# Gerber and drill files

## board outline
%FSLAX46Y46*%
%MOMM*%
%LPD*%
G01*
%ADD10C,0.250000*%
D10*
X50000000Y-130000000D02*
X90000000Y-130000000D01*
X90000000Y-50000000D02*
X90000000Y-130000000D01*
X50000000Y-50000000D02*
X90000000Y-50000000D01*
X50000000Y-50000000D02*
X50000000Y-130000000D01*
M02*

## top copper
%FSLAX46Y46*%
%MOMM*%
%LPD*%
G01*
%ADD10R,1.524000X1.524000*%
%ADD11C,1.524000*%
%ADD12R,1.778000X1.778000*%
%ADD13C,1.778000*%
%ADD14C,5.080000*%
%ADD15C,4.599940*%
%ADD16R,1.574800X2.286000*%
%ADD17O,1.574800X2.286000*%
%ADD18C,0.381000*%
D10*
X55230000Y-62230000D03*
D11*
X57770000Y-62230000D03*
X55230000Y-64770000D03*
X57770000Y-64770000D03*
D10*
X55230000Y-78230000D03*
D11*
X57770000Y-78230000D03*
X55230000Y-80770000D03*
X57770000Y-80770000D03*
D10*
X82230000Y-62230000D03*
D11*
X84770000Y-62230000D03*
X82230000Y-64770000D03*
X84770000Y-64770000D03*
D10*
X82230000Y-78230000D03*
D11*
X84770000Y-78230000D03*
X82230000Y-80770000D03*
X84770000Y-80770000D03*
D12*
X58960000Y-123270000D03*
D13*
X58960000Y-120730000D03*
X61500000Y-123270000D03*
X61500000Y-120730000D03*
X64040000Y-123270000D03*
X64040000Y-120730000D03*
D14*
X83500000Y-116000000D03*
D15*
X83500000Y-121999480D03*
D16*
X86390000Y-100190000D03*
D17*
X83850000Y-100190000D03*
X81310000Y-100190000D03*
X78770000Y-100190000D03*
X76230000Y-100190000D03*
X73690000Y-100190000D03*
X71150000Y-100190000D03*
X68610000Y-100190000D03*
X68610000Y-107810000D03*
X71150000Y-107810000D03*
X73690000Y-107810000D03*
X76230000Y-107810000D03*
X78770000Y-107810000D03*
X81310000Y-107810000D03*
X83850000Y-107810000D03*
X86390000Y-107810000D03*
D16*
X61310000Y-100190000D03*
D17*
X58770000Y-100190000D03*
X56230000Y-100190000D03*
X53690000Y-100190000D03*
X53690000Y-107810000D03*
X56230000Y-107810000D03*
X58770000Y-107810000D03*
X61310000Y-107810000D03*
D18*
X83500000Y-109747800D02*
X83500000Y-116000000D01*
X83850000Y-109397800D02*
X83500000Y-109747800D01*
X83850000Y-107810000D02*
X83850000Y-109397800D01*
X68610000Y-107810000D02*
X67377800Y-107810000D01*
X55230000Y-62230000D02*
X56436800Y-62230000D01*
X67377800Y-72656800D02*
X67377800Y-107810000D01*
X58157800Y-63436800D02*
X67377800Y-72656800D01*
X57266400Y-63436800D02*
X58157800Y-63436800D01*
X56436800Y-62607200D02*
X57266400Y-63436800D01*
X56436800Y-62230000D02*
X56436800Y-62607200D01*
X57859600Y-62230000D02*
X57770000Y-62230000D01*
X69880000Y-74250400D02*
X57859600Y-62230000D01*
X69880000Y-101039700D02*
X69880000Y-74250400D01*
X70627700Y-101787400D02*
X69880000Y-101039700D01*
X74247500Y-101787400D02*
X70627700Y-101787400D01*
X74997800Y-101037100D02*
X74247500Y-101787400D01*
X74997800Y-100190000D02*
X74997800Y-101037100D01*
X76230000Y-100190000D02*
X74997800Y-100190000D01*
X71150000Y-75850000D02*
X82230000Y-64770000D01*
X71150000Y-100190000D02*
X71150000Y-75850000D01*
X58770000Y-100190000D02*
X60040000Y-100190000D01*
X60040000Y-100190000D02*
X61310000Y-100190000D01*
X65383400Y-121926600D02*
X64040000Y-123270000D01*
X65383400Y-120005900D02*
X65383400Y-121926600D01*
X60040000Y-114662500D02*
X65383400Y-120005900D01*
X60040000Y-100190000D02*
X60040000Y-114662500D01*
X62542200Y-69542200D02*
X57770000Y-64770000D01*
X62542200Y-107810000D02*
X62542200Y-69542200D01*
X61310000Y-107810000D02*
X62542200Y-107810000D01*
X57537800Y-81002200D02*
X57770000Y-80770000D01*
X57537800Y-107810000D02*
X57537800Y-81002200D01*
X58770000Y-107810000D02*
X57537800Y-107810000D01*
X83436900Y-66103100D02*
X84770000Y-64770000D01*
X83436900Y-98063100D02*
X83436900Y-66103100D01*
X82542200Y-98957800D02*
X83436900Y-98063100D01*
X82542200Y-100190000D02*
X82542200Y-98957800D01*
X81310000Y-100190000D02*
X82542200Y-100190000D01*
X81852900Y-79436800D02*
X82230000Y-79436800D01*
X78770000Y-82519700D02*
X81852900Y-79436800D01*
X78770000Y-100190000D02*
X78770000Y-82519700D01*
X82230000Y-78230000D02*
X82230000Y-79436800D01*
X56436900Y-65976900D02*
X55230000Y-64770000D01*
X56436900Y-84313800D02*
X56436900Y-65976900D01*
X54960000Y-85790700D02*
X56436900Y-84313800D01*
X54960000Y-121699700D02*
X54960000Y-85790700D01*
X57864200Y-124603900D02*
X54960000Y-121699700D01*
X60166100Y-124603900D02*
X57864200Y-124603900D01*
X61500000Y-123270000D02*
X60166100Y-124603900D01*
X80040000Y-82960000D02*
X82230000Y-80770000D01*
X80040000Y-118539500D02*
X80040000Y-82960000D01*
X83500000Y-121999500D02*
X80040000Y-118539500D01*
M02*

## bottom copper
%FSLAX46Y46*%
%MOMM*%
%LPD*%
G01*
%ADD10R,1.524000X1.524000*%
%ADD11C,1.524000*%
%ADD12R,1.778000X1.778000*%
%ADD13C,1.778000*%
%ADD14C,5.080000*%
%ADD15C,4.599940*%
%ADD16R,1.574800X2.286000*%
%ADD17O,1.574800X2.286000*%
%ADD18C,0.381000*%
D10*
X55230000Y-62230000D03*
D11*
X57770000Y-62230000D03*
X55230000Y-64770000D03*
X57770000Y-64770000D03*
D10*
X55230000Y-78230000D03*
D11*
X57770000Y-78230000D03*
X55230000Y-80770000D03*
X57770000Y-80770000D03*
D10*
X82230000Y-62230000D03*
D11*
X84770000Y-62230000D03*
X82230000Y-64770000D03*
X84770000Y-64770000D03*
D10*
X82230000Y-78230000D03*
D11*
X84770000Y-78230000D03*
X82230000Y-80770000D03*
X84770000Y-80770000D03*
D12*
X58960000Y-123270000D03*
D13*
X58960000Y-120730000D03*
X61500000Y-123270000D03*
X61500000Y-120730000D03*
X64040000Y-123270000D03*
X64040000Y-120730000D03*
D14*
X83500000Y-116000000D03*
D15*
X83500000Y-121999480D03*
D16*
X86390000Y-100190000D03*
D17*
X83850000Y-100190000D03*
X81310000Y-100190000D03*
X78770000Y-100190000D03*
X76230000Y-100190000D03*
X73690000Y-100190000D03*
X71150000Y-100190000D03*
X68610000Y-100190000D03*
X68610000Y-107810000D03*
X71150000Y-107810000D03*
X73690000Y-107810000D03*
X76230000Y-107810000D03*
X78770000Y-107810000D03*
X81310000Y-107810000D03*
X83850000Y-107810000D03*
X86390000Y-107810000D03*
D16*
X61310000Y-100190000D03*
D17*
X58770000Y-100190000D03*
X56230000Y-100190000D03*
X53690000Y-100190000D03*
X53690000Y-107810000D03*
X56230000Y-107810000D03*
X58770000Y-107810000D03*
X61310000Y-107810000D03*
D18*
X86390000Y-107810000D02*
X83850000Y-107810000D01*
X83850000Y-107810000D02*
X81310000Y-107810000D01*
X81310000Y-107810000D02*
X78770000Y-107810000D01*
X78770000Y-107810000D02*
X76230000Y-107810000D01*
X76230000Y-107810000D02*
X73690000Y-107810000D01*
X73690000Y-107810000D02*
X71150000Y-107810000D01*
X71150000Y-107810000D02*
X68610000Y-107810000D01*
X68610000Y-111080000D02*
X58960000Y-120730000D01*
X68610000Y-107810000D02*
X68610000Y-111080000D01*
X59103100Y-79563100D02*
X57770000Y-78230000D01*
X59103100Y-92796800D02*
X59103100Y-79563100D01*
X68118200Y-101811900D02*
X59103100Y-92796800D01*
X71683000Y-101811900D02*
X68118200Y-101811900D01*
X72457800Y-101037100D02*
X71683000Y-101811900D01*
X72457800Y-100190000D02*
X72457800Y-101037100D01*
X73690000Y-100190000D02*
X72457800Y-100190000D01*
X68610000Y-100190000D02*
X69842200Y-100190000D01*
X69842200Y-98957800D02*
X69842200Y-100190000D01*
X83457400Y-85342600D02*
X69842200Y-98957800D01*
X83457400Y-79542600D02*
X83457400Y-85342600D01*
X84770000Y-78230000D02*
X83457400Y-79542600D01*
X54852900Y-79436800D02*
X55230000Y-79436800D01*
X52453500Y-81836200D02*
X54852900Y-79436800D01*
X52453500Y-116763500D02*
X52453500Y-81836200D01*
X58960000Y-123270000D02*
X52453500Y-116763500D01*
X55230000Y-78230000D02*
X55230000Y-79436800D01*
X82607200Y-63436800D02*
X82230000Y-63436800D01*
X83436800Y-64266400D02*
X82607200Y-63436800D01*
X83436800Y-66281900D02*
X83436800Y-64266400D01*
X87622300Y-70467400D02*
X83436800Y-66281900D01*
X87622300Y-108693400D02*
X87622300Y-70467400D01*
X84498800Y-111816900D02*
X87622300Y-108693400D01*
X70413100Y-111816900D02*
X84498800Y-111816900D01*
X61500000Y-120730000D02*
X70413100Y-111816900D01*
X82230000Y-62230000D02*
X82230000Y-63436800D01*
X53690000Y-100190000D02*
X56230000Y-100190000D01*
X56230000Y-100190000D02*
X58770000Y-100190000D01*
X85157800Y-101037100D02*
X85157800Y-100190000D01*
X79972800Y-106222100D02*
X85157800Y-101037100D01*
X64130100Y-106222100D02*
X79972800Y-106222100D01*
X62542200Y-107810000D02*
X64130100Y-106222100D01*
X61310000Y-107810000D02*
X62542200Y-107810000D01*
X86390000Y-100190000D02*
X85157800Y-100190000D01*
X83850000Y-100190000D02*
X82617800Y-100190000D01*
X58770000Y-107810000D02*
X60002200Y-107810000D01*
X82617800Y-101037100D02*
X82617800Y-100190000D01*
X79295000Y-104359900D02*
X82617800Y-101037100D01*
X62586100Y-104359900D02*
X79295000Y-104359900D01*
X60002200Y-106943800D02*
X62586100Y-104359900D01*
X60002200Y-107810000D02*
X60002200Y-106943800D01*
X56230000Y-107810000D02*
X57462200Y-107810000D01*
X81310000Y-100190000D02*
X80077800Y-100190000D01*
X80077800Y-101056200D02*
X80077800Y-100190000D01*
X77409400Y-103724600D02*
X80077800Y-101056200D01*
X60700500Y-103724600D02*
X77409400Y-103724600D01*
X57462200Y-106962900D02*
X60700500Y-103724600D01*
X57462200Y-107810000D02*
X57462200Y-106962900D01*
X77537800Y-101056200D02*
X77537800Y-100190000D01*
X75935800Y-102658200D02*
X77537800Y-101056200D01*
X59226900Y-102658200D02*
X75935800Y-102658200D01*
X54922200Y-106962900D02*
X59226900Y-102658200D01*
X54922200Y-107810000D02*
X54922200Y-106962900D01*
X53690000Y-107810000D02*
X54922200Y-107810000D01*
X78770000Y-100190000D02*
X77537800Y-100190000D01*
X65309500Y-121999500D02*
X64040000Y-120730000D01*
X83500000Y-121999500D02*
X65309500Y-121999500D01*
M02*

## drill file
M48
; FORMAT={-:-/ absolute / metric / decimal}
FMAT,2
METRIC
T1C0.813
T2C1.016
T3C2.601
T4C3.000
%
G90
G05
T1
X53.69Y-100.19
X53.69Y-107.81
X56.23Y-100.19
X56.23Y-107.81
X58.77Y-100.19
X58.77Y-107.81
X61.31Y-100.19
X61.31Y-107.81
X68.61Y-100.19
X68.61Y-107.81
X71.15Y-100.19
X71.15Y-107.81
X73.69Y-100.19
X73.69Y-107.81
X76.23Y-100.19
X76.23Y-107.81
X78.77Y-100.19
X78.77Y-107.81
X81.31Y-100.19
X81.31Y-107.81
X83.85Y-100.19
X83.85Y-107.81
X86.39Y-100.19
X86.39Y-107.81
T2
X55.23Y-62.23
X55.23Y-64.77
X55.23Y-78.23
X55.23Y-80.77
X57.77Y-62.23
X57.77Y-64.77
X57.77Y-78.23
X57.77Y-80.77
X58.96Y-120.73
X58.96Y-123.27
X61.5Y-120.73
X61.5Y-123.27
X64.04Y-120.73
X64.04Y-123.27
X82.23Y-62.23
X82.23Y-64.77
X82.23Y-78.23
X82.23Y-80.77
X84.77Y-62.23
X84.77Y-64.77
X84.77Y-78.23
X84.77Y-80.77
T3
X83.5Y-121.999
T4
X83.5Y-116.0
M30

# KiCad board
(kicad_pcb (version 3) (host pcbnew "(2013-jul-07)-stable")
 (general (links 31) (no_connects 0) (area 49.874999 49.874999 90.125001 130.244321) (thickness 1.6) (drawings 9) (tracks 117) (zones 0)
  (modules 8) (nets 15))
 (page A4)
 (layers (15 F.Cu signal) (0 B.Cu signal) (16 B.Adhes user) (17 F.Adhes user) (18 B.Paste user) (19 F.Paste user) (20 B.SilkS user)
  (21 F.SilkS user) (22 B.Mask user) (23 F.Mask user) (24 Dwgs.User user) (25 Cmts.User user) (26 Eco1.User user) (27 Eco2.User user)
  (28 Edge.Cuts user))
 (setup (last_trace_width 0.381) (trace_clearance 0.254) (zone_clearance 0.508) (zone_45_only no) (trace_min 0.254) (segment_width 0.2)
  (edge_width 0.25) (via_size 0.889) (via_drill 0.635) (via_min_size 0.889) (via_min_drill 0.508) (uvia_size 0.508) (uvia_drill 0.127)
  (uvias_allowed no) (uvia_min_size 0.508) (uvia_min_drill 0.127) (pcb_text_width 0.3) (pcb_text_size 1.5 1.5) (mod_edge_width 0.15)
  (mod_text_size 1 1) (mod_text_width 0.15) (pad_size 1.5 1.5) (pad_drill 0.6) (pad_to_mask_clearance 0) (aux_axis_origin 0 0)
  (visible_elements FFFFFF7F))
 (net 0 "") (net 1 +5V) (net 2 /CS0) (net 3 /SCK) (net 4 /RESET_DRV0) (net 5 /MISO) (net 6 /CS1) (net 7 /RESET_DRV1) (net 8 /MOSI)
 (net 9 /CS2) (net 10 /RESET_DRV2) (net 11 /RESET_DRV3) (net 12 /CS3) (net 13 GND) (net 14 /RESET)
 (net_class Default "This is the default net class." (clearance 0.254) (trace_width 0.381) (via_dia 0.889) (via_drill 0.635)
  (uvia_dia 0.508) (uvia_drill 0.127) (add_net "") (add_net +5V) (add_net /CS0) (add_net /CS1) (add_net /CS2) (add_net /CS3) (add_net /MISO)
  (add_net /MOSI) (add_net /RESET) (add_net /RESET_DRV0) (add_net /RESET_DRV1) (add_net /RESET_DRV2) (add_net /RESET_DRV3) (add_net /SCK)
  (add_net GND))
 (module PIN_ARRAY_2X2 (layer F.Cu) (at 56.5 63.5 270)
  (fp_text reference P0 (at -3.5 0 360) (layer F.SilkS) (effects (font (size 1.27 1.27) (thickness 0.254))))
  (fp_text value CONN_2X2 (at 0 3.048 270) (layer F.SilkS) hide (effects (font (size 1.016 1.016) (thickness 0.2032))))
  (pad 1 thru_hole rect (at -1.27 1.27 270) (size 1.524 1.524) (drill 1.016) (layers *.Cu *.Mask F.SilkS) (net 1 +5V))
  (pad 2 thru_hole circle (at -1.27 -1.27 270) (size 1.524 1.524) (drill 1.016) (layers *.Cu *.Mask F.SilkS) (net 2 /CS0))
  (pad 3 thru_hole circle (at 1.27 1.27 270) (size 1.524 1.524) (drill 1.016) (layers *.Cu *.Mask F.SilkS) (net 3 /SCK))
  (pad 4 thru_hole circle (at 1.27 -1.27 270) (size 1.524 1.524) (drill 1.016) (layers *.Cu *.Mask F.SilkS) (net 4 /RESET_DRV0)))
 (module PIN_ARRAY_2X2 (layer F.Cu) (at 56.5 79.5 270)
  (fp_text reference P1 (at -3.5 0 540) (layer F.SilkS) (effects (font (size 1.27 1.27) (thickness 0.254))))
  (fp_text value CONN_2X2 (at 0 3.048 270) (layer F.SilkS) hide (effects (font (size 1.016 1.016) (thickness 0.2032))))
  (pad 1 thru_hole rect (at -1.27 1.27 270) (size 1.524 1.524) (drill 1.016) (layers *.Cu *.Mask F.SilkS) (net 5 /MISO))
  (pad 2 thru_hole circle (at -1.27 -1.27 270) (size 1.524 1.524) (drill 1.016) (layers *.Cu *.Mask F.SilkS) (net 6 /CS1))
  (pad 3 thru_hole circle (at 1.27 1.27 270) (size 1.524 1.524) (drill 1.016) (layers *.Cu *.Mask F.SilkS))
  (pad 4 thru_hole circle (at 1.27 -1.27 270) (size 1.524 1.524) (drill 1.016) (layers *.Cu *.Mask F.SilkS) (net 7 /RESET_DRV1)))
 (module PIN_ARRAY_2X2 (layer F.Cu) (at 83.5 63.5 270)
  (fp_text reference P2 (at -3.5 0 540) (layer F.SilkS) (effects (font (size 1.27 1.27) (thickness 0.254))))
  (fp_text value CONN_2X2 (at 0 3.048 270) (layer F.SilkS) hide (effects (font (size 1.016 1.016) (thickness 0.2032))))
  (pad 1 thru_hole rect (at -1.27 1.27 270) (size 1.524 1.524) (drill 1.016) (layers *.Cu *.Mask F.SilkS) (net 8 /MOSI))
  (pad 2 thru_hole circle (at -1.27 -1.27 270) (size 1.524 1.524) (drill 1.016) (layers *.Cu *.Mask F.SilkS))
  (pad 3 thru_hole circle (at 1.27 1.27 270) (size 1.524 1.524) (drill 1.016) (layers *.Cu *.Mask F.SilkS) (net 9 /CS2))
  (pad 4 thru_hole circle (at 1.27 -1.27 270) (size 1.524 1.524) (drill 1.016) (layers *.Cu *.Mask F.SilkS) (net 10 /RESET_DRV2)))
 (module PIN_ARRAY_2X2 (layer F.Cu) (at 83.5 79.5 270)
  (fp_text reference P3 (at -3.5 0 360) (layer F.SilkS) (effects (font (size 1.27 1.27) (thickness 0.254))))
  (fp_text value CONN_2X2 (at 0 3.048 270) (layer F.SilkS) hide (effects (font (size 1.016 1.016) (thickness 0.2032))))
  (pad 1 thru_hole rect (at -1.27 1.27 270) (size 1.524 1.524) (drill 1.016) (layers *.Cu *.Mask F.SilkS) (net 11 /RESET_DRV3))
  (pad 2 thru_hole circle (at -1.27 -1.27 270) (size 1.524 1.524) (drill 1.016) (layers *.Cu *.Mask F.SilkS) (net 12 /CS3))
  (pad 3 thru_hole circle (at 1.27 1.27 270) (size 1.524 1.524) (drill 1.016) (layers *.Cu *.Mask F.SilkS) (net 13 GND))
  (pad 4 thru_hole circle (at 1.27 -1.27 270) (size 1.524 1.524) (drill 1.016) (layers *.Cu *.Mask F.SilkS)))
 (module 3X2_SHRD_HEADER (layer F.Cu) (at 61.5 122)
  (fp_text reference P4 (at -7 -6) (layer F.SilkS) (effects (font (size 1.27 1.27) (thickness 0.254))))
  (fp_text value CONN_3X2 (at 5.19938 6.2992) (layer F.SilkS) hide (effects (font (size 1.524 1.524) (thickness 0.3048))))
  (pad 1 thru_hole rect (at -2.54 1.27) (size 1.778 1.778) (drill 1.016) (layers *.Cu *.Mask F.SilkS) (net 5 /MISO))
  (pad 2 thru_hole circle (at -2.54 -1.27) (size 1.778 1.778) (drill 1.016) (layers *.Cu *.Mask F.SilkS) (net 1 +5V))
  (pad 3 thru_hole circle (at 0 1.27) (size 1.778 1.778) (drill 1.016) (layers *.Cu *.Mask F.SilkS) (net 3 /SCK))
  (pad 4 thru_hole circle (at 0 -1.27) (size 1.778 1.778) (drill 1.016) (layers *.Cu *.Mask F.SilkS) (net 8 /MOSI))
  (pad 5 thru_hole circle (at 2.54 1.27) (size 1.778 1.778) (drill 1.016) (layers *.Cu *.Mask F.SilkS) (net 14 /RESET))
  (pad 6 thru_hole circle (at 2.54 -1.27) (size 1.778 1.778) (drill 1.016) (layers *.Cu *.Mask F.SilkS) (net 13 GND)))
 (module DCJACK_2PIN (layer F.Cu) (at 83.5 116 270)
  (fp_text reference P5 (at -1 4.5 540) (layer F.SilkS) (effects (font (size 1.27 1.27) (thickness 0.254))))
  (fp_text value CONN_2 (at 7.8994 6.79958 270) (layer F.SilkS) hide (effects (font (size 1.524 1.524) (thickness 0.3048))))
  (pad 1 thru_hole circle (at 0 0 270) (size 5.08 5.08) (drill 2.99974) (layers *.Cu *.Mask F.SilkS) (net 1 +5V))
  (pad 2 thru_hole circle (at 5.99948 0 270) (size 4.59994 4.59994) (drill 2.60096) (layers *.Cu *.Mask F.SilkS) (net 13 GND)))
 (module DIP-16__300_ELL (layer F.Cu) (at 77.5 104 180)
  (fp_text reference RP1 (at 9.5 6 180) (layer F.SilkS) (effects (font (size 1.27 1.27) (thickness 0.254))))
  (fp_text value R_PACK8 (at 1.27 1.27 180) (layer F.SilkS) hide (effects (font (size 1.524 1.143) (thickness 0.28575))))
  (pad 1 thru_hole rect (at -8.89 3.81 180) (size 1.5748 2.286) (drill 0.8128) (layers *.Cu *.Mask F.SilkS) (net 4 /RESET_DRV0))
  (pad 2 thru_hole oval (at -6.35 3.81 180) (size 1.5748 2.286) (drill 0.8128) (layers *.Cu *.Mask F.SilkS) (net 7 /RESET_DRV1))
  (pad 3 thru_hole oval (at -3.81 3.81 180) (size 1.5748 2.286) (drill 0.8128) (layers *.Cu *.Mask F.SilkS) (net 10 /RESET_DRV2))
  (pad 4 thru_hole oval (at -1.27 3.81 180) (size 1.5748 2.286) (drill 0.8128) (layers *.Cu *.Mask F.SilkS) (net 11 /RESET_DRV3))
  (pad 5 thru_hole oval (at 1.27 3.81 180) (size 1.5748 2.286) (drill 0.8128) (layers *.Cu *.Mask F.SilkS) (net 2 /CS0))
  (pad 6 thru_hole oval (at 3.81 3.81 180) (size 1.5748 2.286) (drill 0.8128) (layers *.Cu *.Mask F.SilkS) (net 6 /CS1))
  (pad 7 thru_hole oval (at 6.35 3.81 180) (size 1.5748 2.286) (drill 0.8128) (layers *.Cu *.Mask F.SilkS) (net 9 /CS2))
  (pad 8 thru_hole oval (at 8.89 3.81 180) (size 1.5748 2.286) (drill 0.8128) (layers *.Cu *.Mask F.SilkS) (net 12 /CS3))
  (pad 9 thru_hole oval (at 8.89 -3.81 180) (size 1.5748 2.286) (drill 0.8128) (layers *.Cu *.Mask F.SilkS) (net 1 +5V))
  (pad 10 thru_hole oval (at 6.35 -3.81 180) (size 1.5748 2.286) (drill 0.8128) (layers *.Cu *.Mask F.SilkS) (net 1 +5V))
  (pad 11 thru_hole oval (at 3.81 -3.81 180) (size 1.5748 2.286) (drill 0.8128) (layers *.Cu *.Mask F.SilkS) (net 1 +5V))
  (pad 12 thru_hole oval (at 1.27 -3.81 180) (size 1.5748 2.286) (drill 0.8128) (layers *.Cu *.Mask F.SilkS) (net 1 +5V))
  (pad 13 thru_hole oval (at -1.27 -3.81 180) (size 1.5748 2.286) (drill 0.8128) (layers *.Cu *.Mask F.SilkS) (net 1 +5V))
  (pad 14 thru_hole oval (at -3.81 -3.81 180) (size 1.5748 2.286) (drill 0.8128) (layers *.Cu *.Mask F.SilkS) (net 1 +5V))
  (pad 15 thru_hole oval (at -6.35 -3.81 180) (size 1.5748 2.286) (drill 0.8128) (layers *.Cu *.Mask F.SilkS) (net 1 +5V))
  (pad 16 thru_hole oval (at -8.89 -3.81 180) (size 1.5748 2.286) (drill 0.8128) (layers *.Cu *.Mask F.SilkS) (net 1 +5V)))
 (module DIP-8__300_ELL (layer F.Cu) (at 57.5 104 180)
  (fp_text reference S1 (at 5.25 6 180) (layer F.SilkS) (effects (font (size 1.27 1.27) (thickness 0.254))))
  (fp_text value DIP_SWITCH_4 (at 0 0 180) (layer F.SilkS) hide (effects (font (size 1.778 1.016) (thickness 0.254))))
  (pad 1 thru_hole rect (at -3.81 3.81 180) (size 1.5748 2.286) (drill 0.8128) (layers *.Cu *.Mask F.SilkS) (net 14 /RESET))
  (pad 2 thru_hole oval (at -1.27 3.81 180) (size 1.5748 2.286) (drill 0.8128) (layers *.Cu *.Mask F.SilkS) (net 14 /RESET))
  (pad 3 thru_hole oval (at 1.27 3.81 180) (size 1.5748 2.286) (drill 0.8128) (layers *.Cu *.Mask F.SilkS) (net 14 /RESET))
  (pad 4 thru_hole oval (at 3.81 3.81 180) (size 1.5748 2.286) (drill 0.8128) (layers *.Cu *.Mask F.SilkS) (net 14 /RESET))
  (pad 5 thru_hole oval (at 3.81 -3.81 180) (size 1.5748 2.286) (drill 0.8128) (layers *.Cu *.Mask F.SilkS) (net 11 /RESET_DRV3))
  (pad 6 thru_hole oval (at 1.27 -3.81 180) (size 1.5748 2.286) (drill 0.8128) (layers *.Cu *.Mask F.SilkS) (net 10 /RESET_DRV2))
  (pad 7 thru_hole oval (at -1.27 -3.81 180) (size 1.5748 2.286) (drill 0.8128) (layers *.Cu *.Mask F.SilkS) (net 7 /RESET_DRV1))
  (pad 8 thru_hole oval (at -3.81 -3.81 180) (size 1.5748 2.286) (drill 0.8128) (layers *.Cu *.Mask F.SilkS) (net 4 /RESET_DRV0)))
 (gr_line (start 50 130) (end 90 130) (angle 90) (layer Edge.Cuts) (width 0.25))
 (gr_line (start 90 50) (end 90 130) (angle 90) (layer Edge.Cuts) (width 0.25))
 (gr_line (start 50 50) (end 90 50) (angle 90) (layer Edge.Cuts) (width 0.25))
 (gr_line (start 50 50) (end 50 130) (angle 90) (layer Edge.Cuts) (width 0.25))
 (segment (start 86.39 107.81) (end 83.85 107.81) (width 0.381) (layer B.Cu) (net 1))
 (segment (start 83.85 107.81) (end 81.31 107.81) (width 0.381) (layer B.Cu) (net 1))
 (segment (start 81.31 107.81) (end 78.77 107.81) (width 0.381) (layer B.Cu) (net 1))
 (segment (start 78.77 107.81) (end 76.23 107.81) (width 0.381) (layer B.Cu) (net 1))
 (segment (start 76.23 107.81) (end 73.69 107.81) (width 0.381) (layer B.Cu) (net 1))
 (segment (start 73.69 107.81) (end 71.15 107.81) (width 0.381) (layer B.Cu) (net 1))
 (segment (start 83.5 109.7478) (end 83.5 116) (width 0.381) (layer F.Cu) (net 1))
 (segment (start 83.85 109.3978) (end 83.5 109.7478) (width 0.381) (layer F.Cu) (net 1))
 (segment (start 83.85 107.81) (end 83.85 109.3978) (width 0.381) (layer F.Cu) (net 1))
 (segment (start 71.15 107.81) (end 68.61 107.81) (width 0.381) (layer B.Cu) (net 1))
 (segment (start 68.61 111.08) (end 58.96 120.73) (width 0.381) (layer B.Cu) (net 1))
 (segment (start 68.61 107.81) (end 68.61 111.08) (width 0.381) (layer B.Cu) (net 1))
 (segment (start 68.61 107.81) (end 67.3778 107.81) (width 0.381) (layer F.Cu) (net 1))
 (segment (start 55.23 62.23) (end 56.4368 62.23) (width 0.381) (layer F.Cu) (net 1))
 (segment (start 67.3778 72.6568) (end 67.3778 107.81) (width 0.381) (layer F.Cu) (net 1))
 (segment (start 58.1578 63.4368) (end 67.3778 72.6568) (width 0.381) (layer F.Cu) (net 1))
 (segment (start 57.2664 63.4368) (end 58.1578 63.4368) (width 0.381) (layer F.Cu) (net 1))
 (segment (start 56.4368 62.6072) (end 57.2664 63.4368) (width 0.381) (layer F.Cu) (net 1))
 (segment (start 56.4368 62.23) (end 56.4368 62.6072) (width 0.381) (layer F.Cu) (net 1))
 (segment (start 57.8596 62.23) (end 57.77 62.23) (width 0.381) (layer F.Cu) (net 2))
 (segment (start 69.88 74.2504) (end 57.8596 62.23) (width 0.381) (layer F.Cu) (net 2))
 (segment (start 69.88 101.0397) (end 69.88 74.2504) (width 0.381) (layer F.Cu) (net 2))
 (segment (start 70.6277 101.7874) (end 69.88 101.0397) (width 0.381) (layer F.Cu) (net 2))
 (segment (start 74.2475 101.7874) (end 70.6277 101.7874) (width 0.381) (layer F.Cu) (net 2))
 (segment (start 74.9978 101.0371) (end 74.2475 101.7874) (width 0.381) (layer F.Cu) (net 2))
 (segment (start 74.9978 100.19) (end 74.9978 101.0371) (width 0.381) (layer F.Cu) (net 2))
 (segment (start 76.23 100.19) (end 74.9978 100.19) (width 0.381) (layer F.Cu) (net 2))
 (segment (start 59.1031 79.5631) (end 57.77 78.23) (width 0.381) (layer B.Cu) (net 6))
 (segment (start 59.1031 92.7968) (end 59.1031 79.5631) (width 0.381) (layer B.Cu) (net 6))
 (segment (start 68.1182 101.8119) (end 59.1031 92.7968) (width 0.381) (layer B.Cu) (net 6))
 (segment (start 71.683 101.8119) (end 68.1182 101.8119) (width 0.381) (layer B.Cu) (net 6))
 (segment (start 72.4578 101.0371) (end 71.683 101.8119) (width 0.381) (layer B.Cu) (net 6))
 (segment (start 72.4578 100.19) (end 72.4578 101.0371) (width 0.381) (layer B.Cu) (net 6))
 (segment (start 73.69 100.19) (end 72.4578 100.19) (width 0.381) (layer B.Cu) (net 6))
 (segment (start 71.15 75.85) (end 82.23 64.77) (width 0.381) (layer F.Cu) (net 9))
 (segment (start 71.15 100.19) (end 71.15 75.85) (width 0.381) (layer F.Cu) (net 9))
 (segment (start 68.61 100.19) (end 69.8422 100.19) (width 0.381) (layer B.Cu) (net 12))
 (segment (start 69.8422 98.9578) (end 69.8422 100.19) (width 0.381) (layer B.Cu) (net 12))
 (segment (start 83.4574 85.3426) (end 69.8422 98.9578) (width 0.381) (layer B.Cu) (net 12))
 (segment (start 83.4574 79.5426) (end 83.4574 85.3426) (width 0.381) (layer B.Cu) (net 12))
 (segment (start 84.77 78.23) (end 83.4574 79.5426) (width 0.381) (layer B.Cu) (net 12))
 (segment (start 54.8529 79.4368) (end 55.23 79.4368) (width 0.381) (layer B.Cu) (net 5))
 (segment (start 52.4535 81.8362) (end 54.8529 79.4368) (width 0.381) (layer B.Cu) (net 5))
 (segment (start 52.4535 116.7635) (end 52.4535 81.8362) (width 0.381) (layer B.Cu) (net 5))
 (segment (start 58.96 123.27) (end 52.4535 116.7635) (width 0.381) (layer B.Cu) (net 5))
 (segment (start 55.23 78.23) (end 55.23 79.4368) (width 0.381) (layer B.Cu) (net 5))
 (segment (start 82.6072 63.4368) (end 82.23 63.4368) (width 0.381) (layer B.Cu) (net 8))
 (segment (start 83.4368 64.2664) (end 82.6072 63.4368) (width 0.381) (layer B.Cu) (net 8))
 (segment (start 83.4368 66.2819) (end 83.4368 64.2664) (width 0.381) (layer B.Cu) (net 8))
 (segment (start 87.6223 70.4674) (end 83.4368 66.2819) (width 0.381) (layer B.Cu) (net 8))
 (segment (start 87.6223 108.6934) (end 87.6223 70.4674) (width 0.381) (layer B.Cu) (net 8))
 (segment (start 84.4988 111.8169) (end 87.6223 108.6934) (width 0.381) (layer B.Cu) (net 8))
 (segment (start 70.4131 111.8169) (end 84.4988 111.8169) (width 0.381) (layer B.Cu) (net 8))
 (segment (start 61.5 120.73) (end 70.4131 111.8169) (width 0.381) (layer B.Cu) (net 8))
 (segment (start 82.23 62.23) (end 82.23 63.4368) (width 0.381) (layer B.Cu) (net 8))
 (segment (start 53.69 100.19) (end 56.23 100.19) (width 0.381) (layer B.Cu) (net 14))
 (segment (start 56.23 100.19) (end 58.77 100.19) (width 0.381) (layer B.Cu) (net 14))
 (segment (start 58.77 100.19) (end 60.04 100.19) (width 0.381) (layer F.Cu) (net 14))
 (segment (start 60.04 100.19) (end 61.31 100.19) (width 0.381) (layer F.Cu) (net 14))
 (segment (start 65.3834 121.9266) (end 64.04 123.27) (width 0.381) (layer F.Cu) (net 14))
 (segment (start 65.3834 120.0059) (end 65.3834 121.9266) (width 0.381) (layer F.Cu) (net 14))
 (segment (start 60.04 114.6625) (end 65.3834 120.0059) (width 0.381) (layer F.Cu) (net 14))
 (segment (start 60.04 100.19) (end 60.04 114.6625) (width 0.381) (layer F.Cu) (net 14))
 (segment (start 62.5422 69.5422) (end 57.77 64.77) (width 0.381) (layer F.Cu) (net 4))
 (segment (start 62.5422 107.81) (end 62.5422 69.5422) (width 0.381) (layer F.Cu) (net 4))
 (segment (start 61.31 107.81) (end 62.5422 107.81) (width 0.381) (layer F.Cu) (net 4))
 (segment (start 85.1578 101.0371) (end 85.1578 100.19) (width 0.381) (layer B.Cu) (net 4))
 (segment (start 79.9728 106.2221) (end 85.1578 101.0371) (width 0.381) (layer B.Cu) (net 4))
 (segment (start 64.1301 106.2221) (end 79.9728 106.2221) (width 0.381) (layer B.Cu) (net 4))
 (segment (start 62.5422 107.81) (end 64.1301 106.2221) (width 0.381) (layer B.Cu) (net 4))
 (segment (start 61.31 107.81) (end 62.5422 107.81) (width 0.381) (layer B.Cu) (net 4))
 (segment (start 86.39 100.19) (end 85.1578 100.19) (width 0.381) (layer B.Cu) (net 4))
 (segment (start 57.5378 81.0022) (end 57.77 80.77) (width 0.381) (layer F.Cu) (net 7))
 (segment (start 57.5378 107.81) (end 57.5378 81.0022) (width 0.381) (layer F.Cu) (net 7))
 (segment (start 58.77 107.81) (end 57.5378 107.81) (width 0.381) (layer F.Cu) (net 7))
 (segment (start 83.85 100.19) (end 82.6178 100.19) (width 0.381) (layer B.Cu) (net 7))
 (segment (start 58.77 107.81) (end 60.0022 107.81) (width 0.381) (layer B.Cu) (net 7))
 (segment (start 82.6178 101.0371) (end 82.6178 100.19) (width 0.381) (layer B.Cu) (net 7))
 (segment (start 79.295 104.3599) (end 82.6178 101.0371) (width 0.381) (layer B.Cu) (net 7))
 (segment (start 62.5861 104.3599) (end 79.295 104.3599) (width 0.381) (layer B.Cu) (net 7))
 (segment (start 60.0022 106.9438) (end 62.5861 104.3599) (width 0.381) (layer B.Cu) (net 7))
 (segment (start 60.0022 107.81) (end 60.0022 106.9438) (width 0.381) (layer B.Cu) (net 7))
 (segment (start 56.23 107.81) (end 57.4622 107.81) (width 0.381) (layer B.Cu) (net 10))
 (segment (start 81.31 100.19) (end 80.0778 100.19) (width 0.381) (layer B.Cu) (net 10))
 (segment (start 83.4369 66.1031) (end 84.77 64.77) (width 0.381) (layer F.Cu) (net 10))
 (segment (start 83.4369 98.0631) (end 83.4369 66.1031) (width 0.381) (layer F.Cu) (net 10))
 (segment (start 82.5422 98.9578) (end 83.4369 98.0631) (width 0.381) (layer F.Cu) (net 10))
 (segment (start 82.5422 100.19) (end 82.5422 98.9578) (width 0.381) (layer F.Cu) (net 10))
 (segment (start 81.31 100.19) (end 82.5422 100.19) (width 0.381) (layer F.Cu) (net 10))
 (segment (start 80.0778 101.0562) (end 80.0778 100.19) (width 0.381) (layer B.Cu) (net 10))
 (segment (start 77.4094 103.7246) (end 80.0778 101.0562) (width 0.381) (layer B.Cu) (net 10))
 (segment (start 60.7005 103.7246) (end 77.4094 103.7246) (width 0.381) (layer B.Cu) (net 10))
 (segment (start 57.4622 106.9629) (end 60.7005 103.7246) (width 0.381) (layer B.Cu) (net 10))
 (segment (start 57.4622 107.81) (end 57.4622 106.9629) (width 0.381) (layer B.Cu) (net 10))
 (segment (start 81.8529 79.4368) (end 82.23 79.4368) (width 0.381) (layer F.Cu) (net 11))
 (segment (start 78.77 82.5197) (end 81.8529 79.4368) (width 0.381) (layer F.Cu) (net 11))
 (segment (start 78.77 100.19) (end 78.77 82.5197) (width 0.381) (layer F.Cu) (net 11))
 (segment (start 82.23 78.23) (end 82.23 79.4368) (width 0.381) (layer F.Cu) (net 11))
 (segment (start 77.5378 101.0562) (end 77.5378 100.19) (width 0.381) (layer B.Cu) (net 11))
 (segment (start 75.9358 102.6582) (end 77.5378 101.0562) (width 0.381) (layer B.Cu) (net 11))
 (segment (start 59.2269 102.6582) (end 75.9358 102.6582) (width 0.381) (layer B.Cu) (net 11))
 (segment (start 54.9222 106.9629) (end 59.2269 102.6582) (width 0.381) (layer B.Cu) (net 11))
 (segment (start 54.9222 107.81) (end 54.9222 106.9629) (width 0.381) (layer B.Cu) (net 11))
 (segment (start 53.69 107.81) (end 54.9222 107.81) (width 0.381) (layer B.Cu) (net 11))
 (segment (start 78.77 100.19) (end 77.5378 100.19) (width 0.381) (layer B.Cu) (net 11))
 (segment (start 56.4369 65.9769) (end 55.23 64.77) (width 0.381) (layer F.Cu) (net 3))
 (segment (start 56.4369 84.3138) (end 56.4369 65.9769) (width 0.381) (layer F.Cu) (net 3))
 (segment (start 54.96 85.7907) (end 56.4369 84.3138) (width 0.381) (layer F.Cu) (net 3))
 (segment (start 54.96 121.6997) (end 54.96 85.7907) (width 0.381) (layer F.Cu) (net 3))
 (segment (start 57.8642 124.6039) (end 54.96 121.6997) (width 0.381) (layer F.Cu) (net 3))
 (segment (start 60.1661 124.6039) (end 57.8642 124.6039) (width 0.381) (layer F.Cu) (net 3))
 (segment (start 61.5 123.27) (end 60.1661 124.6039) (width 0.381) (layer F.Cu) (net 3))
 (segment (start 65.3095 121.9995) (end 64.04 120.73) (width 0.381) (layer B.Cu) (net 13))
 (segment (start 83.5 121.9995) (end 65.3095 121.9995) (width 0.381) (layer B.Cu) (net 13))
 (segment (start 80.04 82.96) (end 82.23 80.77) (width 0.381) (layer F.Cu) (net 13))
 (segment (start 80.04 118.5395) (end 80.04 82.96) (width 0.381) (layer F.Cu) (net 13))
 (segment (start 83.5 121.9995) (end 80.04 118.5395) (width 0.381) (layer F.Cu) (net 13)))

